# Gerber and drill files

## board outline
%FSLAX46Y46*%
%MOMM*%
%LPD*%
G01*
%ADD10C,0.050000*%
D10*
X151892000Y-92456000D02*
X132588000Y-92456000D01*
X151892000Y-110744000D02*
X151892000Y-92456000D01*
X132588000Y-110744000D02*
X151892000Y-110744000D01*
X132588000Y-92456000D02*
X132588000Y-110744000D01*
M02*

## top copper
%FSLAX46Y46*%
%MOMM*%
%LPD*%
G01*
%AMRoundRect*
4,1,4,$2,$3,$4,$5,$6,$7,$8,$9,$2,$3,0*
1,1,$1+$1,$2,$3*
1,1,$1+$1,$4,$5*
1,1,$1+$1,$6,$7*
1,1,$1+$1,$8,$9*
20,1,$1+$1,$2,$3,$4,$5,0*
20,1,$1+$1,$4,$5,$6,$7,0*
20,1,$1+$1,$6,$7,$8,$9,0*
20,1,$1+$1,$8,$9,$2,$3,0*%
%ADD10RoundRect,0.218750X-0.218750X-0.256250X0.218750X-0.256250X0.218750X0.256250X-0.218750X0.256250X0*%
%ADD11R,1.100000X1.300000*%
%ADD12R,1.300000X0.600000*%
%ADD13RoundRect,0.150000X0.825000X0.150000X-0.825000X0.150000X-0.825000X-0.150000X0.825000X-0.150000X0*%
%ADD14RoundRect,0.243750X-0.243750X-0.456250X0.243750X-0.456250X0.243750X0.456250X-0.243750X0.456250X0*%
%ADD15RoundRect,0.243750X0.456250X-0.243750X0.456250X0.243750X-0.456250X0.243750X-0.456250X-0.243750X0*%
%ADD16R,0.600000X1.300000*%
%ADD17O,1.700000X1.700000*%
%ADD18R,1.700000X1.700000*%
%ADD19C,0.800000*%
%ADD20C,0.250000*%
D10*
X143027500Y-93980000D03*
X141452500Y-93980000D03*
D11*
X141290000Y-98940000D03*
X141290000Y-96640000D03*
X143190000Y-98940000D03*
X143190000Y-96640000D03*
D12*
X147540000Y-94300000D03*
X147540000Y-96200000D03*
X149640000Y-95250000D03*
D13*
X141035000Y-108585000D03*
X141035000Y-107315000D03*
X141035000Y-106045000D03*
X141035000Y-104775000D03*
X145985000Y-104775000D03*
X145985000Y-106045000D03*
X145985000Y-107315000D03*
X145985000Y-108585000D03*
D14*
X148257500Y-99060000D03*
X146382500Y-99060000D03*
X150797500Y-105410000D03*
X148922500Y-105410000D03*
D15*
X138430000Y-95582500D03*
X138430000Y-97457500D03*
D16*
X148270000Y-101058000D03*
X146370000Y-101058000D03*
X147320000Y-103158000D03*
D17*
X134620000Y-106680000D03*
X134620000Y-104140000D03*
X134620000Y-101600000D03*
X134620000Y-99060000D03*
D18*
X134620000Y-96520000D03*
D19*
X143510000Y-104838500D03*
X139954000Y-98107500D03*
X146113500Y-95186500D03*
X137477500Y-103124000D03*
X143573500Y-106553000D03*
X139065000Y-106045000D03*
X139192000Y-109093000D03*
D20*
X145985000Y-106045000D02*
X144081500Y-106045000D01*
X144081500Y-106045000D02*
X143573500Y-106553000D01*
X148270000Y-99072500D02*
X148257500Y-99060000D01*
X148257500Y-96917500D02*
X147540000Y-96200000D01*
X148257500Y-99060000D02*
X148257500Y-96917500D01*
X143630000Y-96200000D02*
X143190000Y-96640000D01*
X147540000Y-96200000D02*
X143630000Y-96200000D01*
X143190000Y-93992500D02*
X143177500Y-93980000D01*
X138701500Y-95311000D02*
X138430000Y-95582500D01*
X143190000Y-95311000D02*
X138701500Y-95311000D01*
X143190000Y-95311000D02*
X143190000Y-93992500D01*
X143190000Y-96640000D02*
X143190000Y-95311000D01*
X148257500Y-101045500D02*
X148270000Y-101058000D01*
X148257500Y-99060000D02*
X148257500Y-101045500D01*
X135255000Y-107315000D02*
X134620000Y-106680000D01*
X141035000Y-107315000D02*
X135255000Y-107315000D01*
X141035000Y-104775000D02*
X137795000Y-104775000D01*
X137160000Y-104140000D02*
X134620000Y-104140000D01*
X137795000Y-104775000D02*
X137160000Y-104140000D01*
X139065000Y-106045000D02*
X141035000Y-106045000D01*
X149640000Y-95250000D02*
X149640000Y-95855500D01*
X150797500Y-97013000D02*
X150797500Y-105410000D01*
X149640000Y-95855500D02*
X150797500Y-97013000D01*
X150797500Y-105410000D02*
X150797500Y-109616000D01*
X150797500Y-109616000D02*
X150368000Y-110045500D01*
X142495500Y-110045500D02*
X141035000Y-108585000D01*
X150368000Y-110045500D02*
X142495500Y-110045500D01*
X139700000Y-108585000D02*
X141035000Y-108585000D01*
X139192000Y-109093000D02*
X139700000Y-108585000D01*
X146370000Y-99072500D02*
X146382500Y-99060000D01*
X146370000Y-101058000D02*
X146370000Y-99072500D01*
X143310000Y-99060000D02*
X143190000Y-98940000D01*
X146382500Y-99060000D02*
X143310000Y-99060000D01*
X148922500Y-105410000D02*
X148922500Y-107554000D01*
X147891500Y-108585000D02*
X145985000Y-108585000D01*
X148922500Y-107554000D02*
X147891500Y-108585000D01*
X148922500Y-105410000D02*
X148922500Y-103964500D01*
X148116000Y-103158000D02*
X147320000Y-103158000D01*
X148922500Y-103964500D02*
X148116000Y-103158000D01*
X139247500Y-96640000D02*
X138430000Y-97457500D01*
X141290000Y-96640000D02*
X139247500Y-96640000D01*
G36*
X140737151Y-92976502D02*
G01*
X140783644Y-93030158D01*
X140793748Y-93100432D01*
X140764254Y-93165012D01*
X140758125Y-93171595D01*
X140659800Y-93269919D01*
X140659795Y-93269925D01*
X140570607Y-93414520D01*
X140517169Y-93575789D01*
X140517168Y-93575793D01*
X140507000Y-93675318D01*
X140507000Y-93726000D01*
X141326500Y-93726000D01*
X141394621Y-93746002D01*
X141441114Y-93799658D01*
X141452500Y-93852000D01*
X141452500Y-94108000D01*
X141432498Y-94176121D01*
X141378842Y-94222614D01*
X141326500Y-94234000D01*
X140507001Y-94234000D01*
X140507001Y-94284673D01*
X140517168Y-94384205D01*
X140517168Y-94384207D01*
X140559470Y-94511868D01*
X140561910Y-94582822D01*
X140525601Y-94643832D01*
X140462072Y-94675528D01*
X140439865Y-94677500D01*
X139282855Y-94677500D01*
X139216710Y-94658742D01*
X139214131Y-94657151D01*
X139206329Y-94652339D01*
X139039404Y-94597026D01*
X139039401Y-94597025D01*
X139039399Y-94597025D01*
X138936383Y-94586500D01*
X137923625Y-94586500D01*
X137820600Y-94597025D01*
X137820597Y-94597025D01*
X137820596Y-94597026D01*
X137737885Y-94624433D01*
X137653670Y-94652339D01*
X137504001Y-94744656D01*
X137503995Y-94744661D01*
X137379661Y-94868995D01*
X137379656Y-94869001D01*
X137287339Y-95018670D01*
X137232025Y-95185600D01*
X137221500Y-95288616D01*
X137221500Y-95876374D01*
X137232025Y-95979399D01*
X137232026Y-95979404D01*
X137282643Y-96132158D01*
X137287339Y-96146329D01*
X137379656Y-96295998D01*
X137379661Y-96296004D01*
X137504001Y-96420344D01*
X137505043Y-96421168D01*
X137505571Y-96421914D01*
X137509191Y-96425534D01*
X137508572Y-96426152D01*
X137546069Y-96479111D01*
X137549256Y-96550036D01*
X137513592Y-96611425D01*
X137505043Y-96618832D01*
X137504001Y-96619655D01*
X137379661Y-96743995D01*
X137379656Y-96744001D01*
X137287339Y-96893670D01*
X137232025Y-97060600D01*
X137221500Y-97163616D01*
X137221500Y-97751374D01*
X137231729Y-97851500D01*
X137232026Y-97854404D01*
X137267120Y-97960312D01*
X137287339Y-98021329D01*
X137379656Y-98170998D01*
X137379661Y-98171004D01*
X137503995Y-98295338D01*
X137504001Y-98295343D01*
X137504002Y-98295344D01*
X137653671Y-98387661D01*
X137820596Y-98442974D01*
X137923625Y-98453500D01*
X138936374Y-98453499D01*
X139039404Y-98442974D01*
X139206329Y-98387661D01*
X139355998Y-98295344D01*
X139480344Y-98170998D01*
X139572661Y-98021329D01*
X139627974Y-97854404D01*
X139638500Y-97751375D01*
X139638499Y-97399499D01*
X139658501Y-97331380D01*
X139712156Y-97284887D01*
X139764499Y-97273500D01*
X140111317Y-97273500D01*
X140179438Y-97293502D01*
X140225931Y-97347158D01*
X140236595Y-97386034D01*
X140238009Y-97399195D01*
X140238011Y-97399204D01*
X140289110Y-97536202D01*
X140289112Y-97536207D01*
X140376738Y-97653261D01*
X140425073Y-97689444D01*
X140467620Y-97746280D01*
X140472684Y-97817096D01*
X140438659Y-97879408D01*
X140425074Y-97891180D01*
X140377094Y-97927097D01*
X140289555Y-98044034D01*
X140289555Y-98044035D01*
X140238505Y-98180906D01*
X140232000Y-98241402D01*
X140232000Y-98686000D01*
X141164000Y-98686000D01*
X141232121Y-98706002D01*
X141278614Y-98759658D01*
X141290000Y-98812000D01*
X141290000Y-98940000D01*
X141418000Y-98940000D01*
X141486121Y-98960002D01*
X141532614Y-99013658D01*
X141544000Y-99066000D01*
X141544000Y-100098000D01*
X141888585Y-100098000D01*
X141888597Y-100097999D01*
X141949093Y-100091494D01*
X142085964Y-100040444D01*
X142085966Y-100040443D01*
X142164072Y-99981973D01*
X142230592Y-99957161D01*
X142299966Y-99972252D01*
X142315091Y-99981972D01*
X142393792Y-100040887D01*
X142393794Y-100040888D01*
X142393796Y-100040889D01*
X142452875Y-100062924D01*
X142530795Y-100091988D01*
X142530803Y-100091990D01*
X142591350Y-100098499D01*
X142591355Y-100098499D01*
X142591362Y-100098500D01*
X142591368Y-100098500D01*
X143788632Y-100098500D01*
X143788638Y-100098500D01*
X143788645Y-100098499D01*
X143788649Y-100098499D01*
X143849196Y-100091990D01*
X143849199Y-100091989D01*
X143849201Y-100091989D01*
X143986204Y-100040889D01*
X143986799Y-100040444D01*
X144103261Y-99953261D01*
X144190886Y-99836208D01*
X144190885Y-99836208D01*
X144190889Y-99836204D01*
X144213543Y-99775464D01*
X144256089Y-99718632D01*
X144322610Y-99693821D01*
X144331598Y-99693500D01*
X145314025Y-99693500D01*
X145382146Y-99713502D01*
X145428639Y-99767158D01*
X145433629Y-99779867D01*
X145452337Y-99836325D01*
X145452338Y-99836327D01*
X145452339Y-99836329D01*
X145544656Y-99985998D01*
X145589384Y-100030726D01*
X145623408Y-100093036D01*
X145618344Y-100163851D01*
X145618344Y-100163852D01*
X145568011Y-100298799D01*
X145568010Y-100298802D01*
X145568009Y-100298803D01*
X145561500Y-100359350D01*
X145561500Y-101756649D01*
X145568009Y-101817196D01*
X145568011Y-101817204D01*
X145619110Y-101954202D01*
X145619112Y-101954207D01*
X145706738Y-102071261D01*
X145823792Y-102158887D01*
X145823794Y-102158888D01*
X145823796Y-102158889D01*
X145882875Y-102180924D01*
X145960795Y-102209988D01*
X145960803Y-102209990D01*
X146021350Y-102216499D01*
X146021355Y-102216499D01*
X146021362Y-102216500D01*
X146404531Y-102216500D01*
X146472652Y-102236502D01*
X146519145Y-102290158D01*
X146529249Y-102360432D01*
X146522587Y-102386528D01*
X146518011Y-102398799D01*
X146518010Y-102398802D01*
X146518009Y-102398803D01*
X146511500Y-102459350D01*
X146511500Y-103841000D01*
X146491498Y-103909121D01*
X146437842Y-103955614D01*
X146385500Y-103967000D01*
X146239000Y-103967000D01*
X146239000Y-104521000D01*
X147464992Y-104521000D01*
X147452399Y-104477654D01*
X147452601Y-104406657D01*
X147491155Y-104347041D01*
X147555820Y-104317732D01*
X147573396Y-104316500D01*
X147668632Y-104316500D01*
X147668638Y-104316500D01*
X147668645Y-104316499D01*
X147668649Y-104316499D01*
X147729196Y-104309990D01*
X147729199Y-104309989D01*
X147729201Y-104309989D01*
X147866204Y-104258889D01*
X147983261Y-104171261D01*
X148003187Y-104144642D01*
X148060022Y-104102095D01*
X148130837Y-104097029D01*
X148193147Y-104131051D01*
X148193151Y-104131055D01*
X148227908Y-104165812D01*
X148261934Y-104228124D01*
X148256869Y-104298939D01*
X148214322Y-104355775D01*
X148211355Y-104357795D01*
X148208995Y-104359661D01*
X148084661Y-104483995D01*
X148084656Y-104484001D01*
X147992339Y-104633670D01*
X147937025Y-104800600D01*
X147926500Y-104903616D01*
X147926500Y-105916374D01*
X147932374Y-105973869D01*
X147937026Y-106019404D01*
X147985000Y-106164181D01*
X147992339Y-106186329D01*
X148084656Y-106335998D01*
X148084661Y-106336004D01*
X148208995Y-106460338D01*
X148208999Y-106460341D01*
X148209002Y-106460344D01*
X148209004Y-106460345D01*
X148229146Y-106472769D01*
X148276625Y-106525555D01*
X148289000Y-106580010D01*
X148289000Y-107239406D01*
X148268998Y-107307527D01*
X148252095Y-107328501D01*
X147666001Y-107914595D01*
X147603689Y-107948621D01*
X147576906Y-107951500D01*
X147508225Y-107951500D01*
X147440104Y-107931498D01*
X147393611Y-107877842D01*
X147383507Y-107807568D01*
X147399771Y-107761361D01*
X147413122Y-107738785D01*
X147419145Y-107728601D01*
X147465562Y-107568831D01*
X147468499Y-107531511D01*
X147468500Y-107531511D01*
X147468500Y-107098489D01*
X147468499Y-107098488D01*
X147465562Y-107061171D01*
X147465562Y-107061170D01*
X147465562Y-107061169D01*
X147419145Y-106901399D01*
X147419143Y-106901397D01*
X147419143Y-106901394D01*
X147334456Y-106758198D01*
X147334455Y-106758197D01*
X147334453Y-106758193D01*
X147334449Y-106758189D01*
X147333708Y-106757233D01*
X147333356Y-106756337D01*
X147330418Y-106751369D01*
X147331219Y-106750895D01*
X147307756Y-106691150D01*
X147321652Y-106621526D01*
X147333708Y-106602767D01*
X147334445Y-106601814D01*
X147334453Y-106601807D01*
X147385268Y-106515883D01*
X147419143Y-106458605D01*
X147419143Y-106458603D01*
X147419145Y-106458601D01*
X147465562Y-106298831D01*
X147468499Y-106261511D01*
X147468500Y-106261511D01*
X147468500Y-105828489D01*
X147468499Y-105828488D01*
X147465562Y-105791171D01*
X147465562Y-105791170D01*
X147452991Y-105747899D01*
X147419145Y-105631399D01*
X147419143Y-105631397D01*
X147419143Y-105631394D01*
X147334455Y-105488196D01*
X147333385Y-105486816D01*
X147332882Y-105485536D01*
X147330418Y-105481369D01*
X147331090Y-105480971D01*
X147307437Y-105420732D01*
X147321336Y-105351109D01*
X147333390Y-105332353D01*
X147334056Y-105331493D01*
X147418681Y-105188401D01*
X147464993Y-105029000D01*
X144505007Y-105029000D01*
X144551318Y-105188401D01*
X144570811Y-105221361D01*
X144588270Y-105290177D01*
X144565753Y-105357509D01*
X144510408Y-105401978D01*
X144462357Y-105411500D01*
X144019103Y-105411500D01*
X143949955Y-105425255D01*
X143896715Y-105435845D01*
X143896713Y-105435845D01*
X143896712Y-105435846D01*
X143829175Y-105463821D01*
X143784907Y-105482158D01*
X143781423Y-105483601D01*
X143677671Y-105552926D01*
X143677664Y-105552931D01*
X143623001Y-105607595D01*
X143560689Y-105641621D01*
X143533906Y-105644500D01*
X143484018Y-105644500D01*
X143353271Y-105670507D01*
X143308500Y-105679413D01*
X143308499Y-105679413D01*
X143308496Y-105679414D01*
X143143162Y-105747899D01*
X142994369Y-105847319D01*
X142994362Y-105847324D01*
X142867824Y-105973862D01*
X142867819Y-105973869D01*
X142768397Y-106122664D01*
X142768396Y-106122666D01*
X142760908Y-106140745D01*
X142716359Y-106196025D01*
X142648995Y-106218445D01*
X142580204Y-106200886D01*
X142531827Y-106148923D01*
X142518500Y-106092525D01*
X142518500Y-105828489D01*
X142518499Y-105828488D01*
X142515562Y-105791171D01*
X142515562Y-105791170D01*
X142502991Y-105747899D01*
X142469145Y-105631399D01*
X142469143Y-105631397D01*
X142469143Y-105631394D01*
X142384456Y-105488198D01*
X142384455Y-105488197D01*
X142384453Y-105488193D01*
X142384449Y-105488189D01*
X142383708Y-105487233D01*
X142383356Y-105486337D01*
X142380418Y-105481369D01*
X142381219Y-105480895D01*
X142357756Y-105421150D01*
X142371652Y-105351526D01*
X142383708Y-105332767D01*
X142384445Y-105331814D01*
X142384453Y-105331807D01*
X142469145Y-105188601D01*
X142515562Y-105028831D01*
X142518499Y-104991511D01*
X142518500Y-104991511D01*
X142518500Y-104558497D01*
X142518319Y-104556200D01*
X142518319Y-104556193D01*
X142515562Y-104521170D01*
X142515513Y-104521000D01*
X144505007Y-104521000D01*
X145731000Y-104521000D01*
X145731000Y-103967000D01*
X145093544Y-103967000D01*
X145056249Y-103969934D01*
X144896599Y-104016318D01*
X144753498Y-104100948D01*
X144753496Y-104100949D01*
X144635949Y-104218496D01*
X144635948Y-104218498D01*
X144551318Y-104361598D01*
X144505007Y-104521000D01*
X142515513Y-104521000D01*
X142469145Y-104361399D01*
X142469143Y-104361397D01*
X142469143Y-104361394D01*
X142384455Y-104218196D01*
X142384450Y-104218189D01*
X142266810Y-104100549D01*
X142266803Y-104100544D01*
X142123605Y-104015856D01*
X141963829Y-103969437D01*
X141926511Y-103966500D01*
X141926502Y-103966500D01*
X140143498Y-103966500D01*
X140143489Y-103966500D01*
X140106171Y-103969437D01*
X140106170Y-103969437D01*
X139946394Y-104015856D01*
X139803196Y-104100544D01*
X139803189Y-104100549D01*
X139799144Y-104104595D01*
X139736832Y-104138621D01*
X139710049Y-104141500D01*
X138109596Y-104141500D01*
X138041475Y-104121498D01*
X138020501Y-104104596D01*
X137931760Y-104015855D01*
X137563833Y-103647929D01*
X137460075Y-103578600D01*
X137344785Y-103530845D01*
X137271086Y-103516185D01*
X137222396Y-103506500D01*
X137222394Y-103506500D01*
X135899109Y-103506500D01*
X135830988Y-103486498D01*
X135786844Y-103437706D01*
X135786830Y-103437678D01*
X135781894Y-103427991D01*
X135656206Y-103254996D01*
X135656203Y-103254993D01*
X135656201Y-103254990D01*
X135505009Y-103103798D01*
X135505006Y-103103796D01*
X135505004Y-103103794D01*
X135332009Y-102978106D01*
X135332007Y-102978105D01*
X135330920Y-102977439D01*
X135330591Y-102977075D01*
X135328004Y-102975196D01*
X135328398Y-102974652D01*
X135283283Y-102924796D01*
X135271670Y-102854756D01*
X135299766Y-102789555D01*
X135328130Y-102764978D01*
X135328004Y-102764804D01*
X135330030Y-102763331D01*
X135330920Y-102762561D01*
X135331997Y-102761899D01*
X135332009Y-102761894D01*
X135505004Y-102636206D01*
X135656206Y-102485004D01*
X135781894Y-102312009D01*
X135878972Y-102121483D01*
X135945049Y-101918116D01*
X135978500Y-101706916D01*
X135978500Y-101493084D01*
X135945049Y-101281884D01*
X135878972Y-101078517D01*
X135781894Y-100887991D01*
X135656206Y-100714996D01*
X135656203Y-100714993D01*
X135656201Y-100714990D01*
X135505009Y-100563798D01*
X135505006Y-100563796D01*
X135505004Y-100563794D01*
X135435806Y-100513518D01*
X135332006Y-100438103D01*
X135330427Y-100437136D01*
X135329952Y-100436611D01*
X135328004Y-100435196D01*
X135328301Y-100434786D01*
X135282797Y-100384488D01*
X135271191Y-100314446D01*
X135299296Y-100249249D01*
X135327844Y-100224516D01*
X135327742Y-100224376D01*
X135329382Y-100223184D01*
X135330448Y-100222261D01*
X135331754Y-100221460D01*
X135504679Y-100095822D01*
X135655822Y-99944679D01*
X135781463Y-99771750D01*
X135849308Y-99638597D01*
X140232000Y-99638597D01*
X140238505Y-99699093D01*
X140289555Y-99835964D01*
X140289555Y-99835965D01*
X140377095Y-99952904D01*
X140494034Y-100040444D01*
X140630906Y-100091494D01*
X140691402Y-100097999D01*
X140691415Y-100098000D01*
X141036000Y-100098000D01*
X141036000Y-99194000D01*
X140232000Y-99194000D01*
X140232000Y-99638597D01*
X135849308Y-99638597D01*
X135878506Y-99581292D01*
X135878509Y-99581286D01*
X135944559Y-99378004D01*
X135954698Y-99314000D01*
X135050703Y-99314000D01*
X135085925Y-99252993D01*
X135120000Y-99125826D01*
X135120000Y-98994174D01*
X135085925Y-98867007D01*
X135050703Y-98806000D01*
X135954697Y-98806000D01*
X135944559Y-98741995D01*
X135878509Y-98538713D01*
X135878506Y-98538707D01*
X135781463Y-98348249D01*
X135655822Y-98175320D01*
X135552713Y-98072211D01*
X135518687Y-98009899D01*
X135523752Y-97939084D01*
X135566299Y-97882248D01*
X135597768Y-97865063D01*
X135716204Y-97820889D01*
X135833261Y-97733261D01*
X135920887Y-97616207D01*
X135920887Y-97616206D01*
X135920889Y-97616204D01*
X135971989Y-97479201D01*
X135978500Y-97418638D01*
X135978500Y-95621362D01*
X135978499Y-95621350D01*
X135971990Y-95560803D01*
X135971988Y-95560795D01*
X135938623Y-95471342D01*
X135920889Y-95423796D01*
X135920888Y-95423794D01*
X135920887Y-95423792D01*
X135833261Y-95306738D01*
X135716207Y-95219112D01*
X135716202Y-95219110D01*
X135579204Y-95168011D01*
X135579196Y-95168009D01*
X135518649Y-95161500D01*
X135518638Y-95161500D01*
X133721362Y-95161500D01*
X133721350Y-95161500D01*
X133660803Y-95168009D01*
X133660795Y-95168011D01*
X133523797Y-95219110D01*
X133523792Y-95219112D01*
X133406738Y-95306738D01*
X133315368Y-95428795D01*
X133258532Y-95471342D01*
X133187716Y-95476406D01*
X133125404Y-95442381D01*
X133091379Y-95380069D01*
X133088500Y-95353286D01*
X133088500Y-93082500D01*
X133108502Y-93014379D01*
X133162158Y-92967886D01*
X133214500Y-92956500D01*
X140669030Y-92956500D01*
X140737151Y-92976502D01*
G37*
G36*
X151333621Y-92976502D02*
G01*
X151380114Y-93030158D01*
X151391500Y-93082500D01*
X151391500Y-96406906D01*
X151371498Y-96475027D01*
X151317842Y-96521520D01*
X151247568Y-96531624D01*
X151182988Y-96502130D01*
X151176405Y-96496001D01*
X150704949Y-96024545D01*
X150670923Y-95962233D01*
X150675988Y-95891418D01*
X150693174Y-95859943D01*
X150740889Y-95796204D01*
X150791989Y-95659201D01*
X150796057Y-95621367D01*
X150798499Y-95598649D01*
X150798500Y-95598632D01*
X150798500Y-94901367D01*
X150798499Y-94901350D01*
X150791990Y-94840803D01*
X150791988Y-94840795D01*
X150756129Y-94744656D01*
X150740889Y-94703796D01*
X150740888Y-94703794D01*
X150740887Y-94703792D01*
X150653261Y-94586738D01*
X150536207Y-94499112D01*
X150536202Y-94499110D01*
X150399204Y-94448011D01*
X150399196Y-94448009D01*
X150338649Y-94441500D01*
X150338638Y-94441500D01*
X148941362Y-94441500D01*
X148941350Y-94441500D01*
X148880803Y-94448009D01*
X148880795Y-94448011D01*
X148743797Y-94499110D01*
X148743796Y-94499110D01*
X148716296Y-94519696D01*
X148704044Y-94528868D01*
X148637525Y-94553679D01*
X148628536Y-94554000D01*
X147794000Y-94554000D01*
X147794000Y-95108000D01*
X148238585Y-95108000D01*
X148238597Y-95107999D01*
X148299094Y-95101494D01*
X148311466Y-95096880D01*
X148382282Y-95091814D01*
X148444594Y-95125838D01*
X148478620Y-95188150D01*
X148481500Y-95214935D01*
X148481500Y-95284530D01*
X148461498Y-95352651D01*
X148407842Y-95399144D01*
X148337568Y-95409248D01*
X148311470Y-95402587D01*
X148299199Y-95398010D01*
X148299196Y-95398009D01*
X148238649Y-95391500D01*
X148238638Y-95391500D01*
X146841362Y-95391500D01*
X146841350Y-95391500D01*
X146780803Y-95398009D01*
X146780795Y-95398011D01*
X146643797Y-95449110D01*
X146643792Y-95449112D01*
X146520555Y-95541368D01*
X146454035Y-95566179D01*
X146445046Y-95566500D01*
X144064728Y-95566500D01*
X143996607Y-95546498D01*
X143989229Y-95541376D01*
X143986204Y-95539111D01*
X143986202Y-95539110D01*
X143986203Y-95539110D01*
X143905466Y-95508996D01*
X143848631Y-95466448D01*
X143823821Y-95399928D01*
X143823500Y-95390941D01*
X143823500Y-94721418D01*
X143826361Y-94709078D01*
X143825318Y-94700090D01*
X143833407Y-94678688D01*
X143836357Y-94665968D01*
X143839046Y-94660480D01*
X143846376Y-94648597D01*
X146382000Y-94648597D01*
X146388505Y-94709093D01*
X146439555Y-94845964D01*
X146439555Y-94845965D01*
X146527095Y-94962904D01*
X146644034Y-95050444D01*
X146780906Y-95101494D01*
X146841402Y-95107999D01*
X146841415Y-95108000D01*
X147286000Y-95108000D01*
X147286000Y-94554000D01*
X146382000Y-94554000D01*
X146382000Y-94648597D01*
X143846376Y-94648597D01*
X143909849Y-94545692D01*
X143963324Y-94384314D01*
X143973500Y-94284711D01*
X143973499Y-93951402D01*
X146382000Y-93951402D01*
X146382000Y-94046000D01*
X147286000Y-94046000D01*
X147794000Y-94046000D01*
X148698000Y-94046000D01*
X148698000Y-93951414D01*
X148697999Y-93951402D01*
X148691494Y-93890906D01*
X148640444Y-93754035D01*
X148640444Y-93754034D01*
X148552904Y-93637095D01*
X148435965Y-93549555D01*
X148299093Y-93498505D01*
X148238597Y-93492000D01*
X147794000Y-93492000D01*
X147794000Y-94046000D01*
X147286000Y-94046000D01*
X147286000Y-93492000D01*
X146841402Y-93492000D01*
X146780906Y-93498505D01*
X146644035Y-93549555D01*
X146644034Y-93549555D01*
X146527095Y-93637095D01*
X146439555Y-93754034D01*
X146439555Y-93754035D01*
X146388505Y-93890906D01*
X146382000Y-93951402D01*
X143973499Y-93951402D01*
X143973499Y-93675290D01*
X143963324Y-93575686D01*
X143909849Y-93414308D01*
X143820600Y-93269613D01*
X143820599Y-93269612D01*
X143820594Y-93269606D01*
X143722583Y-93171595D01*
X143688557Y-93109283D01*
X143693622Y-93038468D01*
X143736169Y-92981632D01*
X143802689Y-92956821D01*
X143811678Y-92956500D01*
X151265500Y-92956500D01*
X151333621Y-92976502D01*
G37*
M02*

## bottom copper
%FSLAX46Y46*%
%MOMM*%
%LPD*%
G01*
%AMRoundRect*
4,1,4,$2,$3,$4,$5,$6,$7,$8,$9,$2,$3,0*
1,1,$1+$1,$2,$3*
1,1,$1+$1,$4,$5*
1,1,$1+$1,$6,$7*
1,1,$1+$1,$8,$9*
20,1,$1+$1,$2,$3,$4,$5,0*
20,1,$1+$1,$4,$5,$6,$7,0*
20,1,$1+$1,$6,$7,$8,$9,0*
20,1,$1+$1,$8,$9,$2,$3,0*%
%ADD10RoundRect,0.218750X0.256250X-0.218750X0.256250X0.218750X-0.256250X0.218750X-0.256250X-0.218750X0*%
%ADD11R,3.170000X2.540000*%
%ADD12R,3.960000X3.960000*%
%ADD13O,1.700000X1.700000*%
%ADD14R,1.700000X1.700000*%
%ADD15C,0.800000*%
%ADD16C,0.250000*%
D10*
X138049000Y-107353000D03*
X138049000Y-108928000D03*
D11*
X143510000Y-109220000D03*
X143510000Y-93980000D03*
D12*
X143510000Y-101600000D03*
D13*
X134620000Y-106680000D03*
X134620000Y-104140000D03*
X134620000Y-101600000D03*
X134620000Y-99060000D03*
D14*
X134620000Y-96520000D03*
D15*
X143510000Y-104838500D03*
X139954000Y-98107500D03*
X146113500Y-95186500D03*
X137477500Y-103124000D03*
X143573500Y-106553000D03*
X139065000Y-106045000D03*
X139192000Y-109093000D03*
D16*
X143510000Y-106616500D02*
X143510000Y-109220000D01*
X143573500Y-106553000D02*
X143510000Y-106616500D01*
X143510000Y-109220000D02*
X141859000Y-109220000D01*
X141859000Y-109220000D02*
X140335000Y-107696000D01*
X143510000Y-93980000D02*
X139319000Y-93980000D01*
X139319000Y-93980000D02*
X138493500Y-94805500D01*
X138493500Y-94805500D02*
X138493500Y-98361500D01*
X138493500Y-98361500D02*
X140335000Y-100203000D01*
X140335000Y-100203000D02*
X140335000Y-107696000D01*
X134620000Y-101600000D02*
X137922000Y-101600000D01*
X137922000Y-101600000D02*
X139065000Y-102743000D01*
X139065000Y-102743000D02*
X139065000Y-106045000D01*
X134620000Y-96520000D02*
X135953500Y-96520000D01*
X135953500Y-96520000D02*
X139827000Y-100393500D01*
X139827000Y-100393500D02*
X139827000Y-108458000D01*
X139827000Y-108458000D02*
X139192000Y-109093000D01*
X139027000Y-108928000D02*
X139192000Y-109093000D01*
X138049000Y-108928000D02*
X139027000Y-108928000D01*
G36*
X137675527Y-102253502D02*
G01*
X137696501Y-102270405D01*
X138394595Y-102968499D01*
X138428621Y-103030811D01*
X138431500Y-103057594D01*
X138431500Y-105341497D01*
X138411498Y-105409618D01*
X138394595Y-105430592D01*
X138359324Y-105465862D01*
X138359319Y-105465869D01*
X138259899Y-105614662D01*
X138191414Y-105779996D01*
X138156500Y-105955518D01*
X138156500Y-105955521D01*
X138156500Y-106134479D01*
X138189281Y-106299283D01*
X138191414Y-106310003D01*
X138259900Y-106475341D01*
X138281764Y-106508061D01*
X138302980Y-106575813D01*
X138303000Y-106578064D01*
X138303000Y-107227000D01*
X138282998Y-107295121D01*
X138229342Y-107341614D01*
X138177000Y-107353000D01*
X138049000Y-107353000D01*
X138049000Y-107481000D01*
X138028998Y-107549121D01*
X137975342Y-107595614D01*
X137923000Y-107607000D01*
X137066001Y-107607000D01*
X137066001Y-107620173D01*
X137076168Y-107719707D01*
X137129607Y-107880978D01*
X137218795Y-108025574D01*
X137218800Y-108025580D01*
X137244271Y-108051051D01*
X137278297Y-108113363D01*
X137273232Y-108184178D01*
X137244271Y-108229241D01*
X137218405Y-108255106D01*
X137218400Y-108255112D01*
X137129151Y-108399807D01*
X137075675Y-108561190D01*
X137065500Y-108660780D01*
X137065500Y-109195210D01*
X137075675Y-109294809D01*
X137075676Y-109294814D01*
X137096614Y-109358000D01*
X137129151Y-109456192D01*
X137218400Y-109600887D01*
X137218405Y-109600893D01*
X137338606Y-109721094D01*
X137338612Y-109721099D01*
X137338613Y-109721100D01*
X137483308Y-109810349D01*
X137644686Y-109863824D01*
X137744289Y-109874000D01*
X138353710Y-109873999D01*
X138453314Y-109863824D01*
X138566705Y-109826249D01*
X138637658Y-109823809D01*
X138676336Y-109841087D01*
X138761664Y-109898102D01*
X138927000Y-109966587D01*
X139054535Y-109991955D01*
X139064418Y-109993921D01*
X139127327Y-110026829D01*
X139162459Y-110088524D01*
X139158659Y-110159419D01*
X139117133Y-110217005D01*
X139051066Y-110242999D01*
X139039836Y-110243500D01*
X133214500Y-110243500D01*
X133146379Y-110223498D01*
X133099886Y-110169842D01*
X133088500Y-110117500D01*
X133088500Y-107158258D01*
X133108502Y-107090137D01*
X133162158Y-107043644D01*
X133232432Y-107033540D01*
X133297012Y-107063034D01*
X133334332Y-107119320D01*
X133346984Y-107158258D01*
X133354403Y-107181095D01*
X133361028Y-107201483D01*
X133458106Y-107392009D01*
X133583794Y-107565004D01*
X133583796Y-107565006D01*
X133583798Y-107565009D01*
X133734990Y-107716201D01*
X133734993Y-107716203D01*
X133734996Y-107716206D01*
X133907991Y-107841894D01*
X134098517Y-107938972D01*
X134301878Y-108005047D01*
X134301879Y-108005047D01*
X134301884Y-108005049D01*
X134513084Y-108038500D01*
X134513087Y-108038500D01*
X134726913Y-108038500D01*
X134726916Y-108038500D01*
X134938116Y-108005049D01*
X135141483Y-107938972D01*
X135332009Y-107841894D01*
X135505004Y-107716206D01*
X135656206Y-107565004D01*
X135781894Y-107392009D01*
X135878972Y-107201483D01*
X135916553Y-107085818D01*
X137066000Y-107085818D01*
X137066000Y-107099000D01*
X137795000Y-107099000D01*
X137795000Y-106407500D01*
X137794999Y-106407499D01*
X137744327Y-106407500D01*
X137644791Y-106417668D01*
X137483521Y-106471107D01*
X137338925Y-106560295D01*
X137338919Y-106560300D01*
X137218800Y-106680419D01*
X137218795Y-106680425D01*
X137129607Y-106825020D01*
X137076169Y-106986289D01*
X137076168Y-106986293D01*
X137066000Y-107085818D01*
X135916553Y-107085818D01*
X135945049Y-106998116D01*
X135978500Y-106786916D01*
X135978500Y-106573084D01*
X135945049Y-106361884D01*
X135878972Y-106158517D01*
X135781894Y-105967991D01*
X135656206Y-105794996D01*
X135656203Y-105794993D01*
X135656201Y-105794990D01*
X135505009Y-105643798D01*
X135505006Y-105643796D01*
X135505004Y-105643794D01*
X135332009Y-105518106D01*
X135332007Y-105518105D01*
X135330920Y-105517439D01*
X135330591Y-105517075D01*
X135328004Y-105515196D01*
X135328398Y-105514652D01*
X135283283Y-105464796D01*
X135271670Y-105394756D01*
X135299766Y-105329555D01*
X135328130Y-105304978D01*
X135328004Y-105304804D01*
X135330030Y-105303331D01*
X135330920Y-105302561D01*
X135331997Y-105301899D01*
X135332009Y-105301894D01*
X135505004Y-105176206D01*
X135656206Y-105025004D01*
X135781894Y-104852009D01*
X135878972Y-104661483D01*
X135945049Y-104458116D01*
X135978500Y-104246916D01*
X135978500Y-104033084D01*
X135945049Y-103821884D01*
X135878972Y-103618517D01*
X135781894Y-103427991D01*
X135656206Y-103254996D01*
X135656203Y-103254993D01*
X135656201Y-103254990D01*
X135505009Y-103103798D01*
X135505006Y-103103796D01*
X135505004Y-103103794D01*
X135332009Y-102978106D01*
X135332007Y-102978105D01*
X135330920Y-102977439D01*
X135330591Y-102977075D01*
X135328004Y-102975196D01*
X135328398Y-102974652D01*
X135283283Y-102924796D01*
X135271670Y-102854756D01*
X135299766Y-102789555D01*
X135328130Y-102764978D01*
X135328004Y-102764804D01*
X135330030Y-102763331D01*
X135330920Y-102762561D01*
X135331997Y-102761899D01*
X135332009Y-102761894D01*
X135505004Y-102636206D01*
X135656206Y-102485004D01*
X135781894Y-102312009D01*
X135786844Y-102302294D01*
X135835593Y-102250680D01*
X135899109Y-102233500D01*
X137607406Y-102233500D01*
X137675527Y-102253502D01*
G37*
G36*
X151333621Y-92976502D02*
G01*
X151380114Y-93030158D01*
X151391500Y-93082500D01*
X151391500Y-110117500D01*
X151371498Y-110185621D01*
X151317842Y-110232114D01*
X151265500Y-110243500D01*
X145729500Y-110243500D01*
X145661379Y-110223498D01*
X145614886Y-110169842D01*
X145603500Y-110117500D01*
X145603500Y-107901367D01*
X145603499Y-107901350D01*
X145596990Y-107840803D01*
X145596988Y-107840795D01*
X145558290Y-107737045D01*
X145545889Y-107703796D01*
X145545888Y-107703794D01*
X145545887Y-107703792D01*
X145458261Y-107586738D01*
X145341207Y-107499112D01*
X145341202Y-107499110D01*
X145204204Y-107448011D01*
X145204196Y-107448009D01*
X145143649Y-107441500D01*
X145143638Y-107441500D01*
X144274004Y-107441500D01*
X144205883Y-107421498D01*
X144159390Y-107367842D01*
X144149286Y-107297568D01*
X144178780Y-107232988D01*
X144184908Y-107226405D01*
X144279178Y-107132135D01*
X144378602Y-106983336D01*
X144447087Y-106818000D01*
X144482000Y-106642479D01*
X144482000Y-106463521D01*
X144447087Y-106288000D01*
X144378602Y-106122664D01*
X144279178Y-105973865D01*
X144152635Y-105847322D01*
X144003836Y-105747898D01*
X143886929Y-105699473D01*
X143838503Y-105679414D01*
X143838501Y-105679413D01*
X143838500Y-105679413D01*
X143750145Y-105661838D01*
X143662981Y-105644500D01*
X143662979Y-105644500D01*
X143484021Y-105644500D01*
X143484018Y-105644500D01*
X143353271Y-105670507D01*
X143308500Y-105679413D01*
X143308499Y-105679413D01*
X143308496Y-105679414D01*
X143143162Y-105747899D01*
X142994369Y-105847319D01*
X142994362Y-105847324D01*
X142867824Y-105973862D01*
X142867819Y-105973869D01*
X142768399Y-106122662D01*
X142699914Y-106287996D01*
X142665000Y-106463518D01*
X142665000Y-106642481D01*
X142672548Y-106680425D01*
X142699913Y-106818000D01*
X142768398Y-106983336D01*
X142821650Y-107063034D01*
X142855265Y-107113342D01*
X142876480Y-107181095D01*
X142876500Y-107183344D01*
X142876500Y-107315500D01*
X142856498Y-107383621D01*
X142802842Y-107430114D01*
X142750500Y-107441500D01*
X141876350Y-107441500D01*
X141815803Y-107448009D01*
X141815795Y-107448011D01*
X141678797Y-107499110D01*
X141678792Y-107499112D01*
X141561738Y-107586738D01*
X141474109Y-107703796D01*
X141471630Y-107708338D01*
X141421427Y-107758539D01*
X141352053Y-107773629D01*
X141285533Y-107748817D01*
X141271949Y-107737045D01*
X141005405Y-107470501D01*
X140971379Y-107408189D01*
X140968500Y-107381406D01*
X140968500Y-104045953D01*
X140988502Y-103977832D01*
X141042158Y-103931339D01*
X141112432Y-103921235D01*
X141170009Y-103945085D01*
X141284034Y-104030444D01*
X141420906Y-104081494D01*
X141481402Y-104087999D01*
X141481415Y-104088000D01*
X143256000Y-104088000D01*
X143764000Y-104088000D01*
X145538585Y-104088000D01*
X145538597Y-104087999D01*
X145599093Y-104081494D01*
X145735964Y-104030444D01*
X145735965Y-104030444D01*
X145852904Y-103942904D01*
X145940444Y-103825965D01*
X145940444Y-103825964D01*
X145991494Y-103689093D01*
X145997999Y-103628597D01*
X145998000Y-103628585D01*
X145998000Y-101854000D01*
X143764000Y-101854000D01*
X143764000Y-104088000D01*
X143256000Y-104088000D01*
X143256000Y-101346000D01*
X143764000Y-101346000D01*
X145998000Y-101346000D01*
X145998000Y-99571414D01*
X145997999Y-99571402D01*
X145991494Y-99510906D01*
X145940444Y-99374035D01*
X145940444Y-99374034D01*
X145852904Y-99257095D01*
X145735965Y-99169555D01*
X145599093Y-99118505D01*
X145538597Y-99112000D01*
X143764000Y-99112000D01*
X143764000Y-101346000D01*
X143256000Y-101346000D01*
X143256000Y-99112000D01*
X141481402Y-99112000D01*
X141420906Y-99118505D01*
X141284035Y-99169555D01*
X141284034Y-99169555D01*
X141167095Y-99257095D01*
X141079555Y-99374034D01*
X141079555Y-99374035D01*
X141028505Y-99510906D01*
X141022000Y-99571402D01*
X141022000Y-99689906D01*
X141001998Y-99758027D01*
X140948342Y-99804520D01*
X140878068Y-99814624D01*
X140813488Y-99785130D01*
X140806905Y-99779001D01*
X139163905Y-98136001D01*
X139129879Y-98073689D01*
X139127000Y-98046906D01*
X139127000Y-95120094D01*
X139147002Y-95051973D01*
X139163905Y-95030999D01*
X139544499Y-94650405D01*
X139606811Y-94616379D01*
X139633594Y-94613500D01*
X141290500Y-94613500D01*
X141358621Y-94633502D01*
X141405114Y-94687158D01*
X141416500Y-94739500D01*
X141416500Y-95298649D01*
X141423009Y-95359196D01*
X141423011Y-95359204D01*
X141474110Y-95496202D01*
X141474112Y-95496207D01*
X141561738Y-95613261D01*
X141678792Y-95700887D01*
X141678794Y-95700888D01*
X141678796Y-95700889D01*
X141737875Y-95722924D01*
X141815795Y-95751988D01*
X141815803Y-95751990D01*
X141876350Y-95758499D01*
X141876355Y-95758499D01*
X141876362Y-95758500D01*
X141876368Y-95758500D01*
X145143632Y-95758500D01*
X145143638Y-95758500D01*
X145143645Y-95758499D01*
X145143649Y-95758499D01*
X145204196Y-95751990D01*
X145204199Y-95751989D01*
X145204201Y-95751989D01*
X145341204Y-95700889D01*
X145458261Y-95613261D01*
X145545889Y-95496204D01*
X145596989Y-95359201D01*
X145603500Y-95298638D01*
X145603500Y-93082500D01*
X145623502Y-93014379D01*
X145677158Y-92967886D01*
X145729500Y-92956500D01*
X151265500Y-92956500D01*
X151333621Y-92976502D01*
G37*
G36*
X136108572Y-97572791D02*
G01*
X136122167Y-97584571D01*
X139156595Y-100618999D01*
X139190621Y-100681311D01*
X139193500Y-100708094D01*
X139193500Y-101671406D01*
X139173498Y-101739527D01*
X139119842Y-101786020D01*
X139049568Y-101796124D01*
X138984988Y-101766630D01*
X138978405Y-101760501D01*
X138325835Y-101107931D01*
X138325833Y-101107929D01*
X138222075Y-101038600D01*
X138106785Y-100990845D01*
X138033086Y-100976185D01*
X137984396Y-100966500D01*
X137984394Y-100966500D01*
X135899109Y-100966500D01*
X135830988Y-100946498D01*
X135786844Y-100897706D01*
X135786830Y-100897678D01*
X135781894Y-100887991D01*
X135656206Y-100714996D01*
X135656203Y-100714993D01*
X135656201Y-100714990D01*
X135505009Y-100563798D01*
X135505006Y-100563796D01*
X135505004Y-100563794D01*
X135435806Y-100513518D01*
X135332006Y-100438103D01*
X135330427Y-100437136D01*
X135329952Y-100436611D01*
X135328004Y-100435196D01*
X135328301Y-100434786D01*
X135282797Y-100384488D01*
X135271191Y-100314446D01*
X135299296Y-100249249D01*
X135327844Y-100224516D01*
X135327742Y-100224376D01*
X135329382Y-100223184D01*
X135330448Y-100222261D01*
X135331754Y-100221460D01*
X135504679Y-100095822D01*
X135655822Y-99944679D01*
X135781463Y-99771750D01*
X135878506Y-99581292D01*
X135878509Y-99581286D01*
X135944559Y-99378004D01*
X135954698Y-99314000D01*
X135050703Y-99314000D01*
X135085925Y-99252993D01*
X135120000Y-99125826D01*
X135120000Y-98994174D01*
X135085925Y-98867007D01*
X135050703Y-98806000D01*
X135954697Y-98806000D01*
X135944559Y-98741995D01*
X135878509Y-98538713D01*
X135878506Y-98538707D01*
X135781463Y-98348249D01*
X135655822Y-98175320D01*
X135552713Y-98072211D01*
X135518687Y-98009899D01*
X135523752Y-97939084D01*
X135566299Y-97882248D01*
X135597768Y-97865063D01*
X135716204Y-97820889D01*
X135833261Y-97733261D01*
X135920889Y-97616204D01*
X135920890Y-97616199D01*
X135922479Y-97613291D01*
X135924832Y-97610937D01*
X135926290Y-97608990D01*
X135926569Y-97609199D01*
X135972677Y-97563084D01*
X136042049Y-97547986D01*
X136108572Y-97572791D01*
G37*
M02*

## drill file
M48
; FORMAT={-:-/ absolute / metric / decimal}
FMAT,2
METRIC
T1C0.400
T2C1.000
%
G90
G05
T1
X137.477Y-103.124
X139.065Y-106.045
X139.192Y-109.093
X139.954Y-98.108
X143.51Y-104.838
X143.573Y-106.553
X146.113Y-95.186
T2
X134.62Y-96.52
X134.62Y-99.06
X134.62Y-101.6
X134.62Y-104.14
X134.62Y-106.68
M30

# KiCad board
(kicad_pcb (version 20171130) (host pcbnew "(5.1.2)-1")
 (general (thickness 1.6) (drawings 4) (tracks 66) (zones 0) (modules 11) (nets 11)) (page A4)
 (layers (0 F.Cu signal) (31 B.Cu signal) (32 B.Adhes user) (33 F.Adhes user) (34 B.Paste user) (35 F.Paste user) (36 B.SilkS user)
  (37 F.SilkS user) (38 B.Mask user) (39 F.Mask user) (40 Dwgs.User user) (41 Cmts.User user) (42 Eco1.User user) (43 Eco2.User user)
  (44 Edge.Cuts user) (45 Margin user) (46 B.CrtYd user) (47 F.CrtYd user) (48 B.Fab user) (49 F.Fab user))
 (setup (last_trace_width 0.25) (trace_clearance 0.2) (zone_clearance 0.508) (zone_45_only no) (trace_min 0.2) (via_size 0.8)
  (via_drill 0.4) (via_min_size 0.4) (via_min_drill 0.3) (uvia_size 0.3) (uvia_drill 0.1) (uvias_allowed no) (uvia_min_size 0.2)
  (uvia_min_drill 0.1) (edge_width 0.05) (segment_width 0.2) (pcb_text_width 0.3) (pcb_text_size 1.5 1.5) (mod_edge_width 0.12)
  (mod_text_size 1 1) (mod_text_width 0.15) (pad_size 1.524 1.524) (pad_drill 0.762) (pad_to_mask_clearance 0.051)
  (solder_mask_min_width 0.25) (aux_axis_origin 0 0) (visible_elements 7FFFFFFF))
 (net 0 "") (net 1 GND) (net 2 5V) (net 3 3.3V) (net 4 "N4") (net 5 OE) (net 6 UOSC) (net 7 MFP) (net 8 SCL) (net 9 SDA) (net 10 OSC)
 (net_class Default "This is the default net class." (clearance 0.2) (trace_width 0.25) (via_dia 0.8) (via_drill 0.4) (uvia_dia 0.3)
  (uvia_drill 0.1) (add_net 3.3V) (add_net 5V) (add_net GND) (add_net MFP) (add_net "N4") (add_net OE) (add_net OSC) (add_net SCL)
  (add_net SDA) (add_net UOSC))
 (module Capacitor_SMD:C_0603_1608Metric (layer B.Cu) (at 138.049 108.1405 90)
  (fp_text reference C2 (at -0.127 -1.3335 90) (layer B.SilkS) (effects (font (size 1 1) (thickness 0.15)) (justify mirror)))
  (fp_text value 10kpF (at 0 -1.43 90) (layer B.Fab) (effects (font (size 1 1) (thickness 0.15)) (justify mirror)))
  (pad 2 smd roundrect (at 0.7875 0 90) (size 0.875 0.95) (layers B.Cu B.Paste B.Mask) (roundrect_rratio 0.25) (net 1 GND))
  (pad 1 smd roundrect (at -0.7875 0 90) (size 0.875 0.95) (layers B.Cu B.Paste B.Mask) (roundrect_rratio 0.25) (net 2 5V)))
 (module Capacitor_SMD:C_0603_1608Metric (layer F.Cu) (at 142.24 93.98)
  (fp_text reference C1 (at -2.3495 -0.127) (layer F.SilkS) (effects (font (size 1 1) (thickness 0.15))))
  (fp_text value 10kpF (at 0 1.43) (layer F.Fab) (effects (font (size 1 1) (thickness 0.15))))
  (pad 2 smd roundrect (at 0.7875 0) (size 0.875 0.95) (layers F.Cu F.Paste F.Mask) (roundrect_rratio 0.25) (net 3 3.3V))
  (pad 1 smd roundrect (at -0.7875 0) (size 0.875 0.95) (layers F.Cu F.Paste F.Mask) (roundrect_rratio 0.25) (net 1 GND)))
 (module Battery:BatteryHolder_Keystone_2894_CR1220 (layer B.Cu) (at 143.51 101.6 270)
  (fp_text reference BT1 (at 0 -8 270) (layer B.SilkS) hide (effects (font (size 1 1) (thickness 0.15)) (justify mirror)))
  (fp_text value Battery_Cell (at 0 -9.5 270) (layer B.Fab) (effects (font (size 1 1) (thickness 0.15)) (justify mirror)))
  (pad 1 smd rect (at 7.62 0 270) (size 2.54 3.17) (layers B.Cu B.Paste B.Mask) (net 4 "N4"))
  (pad 1 smd rect (at -7.62 0 270) (size 2.54 3.17) (layers B.Cu B.Paste B.Mask) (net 4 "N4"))
  (pad 2 smd rect (at 0 0 270) (size 3.96 3.96) (layers B.Cu B.Paste B.Mask) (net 1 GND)))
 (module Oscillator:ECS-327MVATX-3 (layer F.Cu) (at 142.24 97.79 270)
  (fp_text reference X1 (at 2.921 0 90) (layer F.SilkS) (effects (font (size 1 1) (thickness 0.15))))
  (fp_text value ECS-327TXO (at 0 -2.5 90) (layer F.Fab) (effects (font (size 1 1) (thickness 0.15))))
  (pad 2 smd rect (at 1.15 0.95 270) (size 1.3 1.1) (layers F.Cu F.Paste F.Mask) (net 1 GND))
  (pad 1 smd rect (at -1.15 0.95 270) (size 1.3 1.1) (layers F.Cu F.Paste F.Mask) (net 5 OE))
  (pad 3 smd rect (at 1.15 -0.95 270) (size 1.3 1.1) (layers F.Cu F.Paste F.Mask) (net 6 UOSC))
  (pad 4 smd rect (at -1.15 -0.95 270) (size 1.3 1.1) (layers F.Cu F.Paste F.Mask) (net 3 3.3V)))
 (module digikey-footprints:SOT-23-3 (layer F.Cu) (at 148.59 95.25)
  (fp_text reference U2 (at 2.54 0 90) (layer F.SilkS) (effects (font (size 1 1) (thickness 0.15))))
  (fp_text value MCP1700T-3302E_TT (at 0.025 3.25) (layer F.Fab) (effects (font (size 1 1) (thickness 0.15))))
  (pad 1 smd rect (at -1.05 -0.95) (size 1.3 0.6) (layers F.Cu F.Paste F.Mask) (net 1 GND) (solder_mask_margin 0.07))
  (pad 2 smd rect (at -1.05 0.95) (size 1.3 0.6) (layers F.Cu F.Paste F.Mask) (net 3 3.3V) (solder_mask_margin 0.07))
  (pad 3 smd rect (at 1.05 0) (size 1.3 0.6) (layers F.Cu F.Paste F.Mask) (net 2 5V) (solder_mask_margin 0.07)))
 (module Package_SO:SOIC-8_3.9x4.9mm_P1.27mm (layer F.Cu) (at 143.51 106.68 180)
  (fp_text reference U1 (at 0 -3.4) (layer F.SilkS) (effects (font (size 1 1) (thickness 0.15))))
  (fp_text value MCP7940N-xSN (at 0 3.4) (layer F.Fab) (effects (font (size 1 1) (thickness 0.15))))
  (pad 8 smd roundrect (at 2.475 -1.905 180) (size 1.95 0.6) (layers F.Cu F.Paste F.Mask) (roundrect_rratio 0.25) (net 2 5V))
  (pad 7 smd roundrect (at 2.475 -0.635 180) (size 1.95 0.6) (layers F.Cu F.Paste F.Mask) (roundrect_rratio 0.25) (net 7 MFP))
  (pad 6 smd roundrect (at 2.475 0.635 180) (size 1.95 0.6) (layers F.Cu F.Paste F.Mask) (roundrect_rratio 0.25) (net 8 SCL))
  (pad 5 smd roundrect (at 2.475 1.905 180) (size 1.95 0.6) (layers F.Cu F.Paste F.Mask) (roundrect_rratio 0.25) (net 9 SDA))
  (pad 4 smd roundrect (at -2.475 1.905 180) (size 1.95 0.6) (layers F.Cu F.Paste F.Mask) (roundrect_rratio 0.25) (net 1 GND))
  (pad 3 smd roundrect (at -2.475 0.635 180) (size 1.95 0.6) (layers F.Cu F.Paste F.Mask) (roundrect_rratio 0.25) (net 4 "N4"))
  (pad 2 smd roundrect (at -2.475 -0.635 180) (size 1.95 0.6) (layers F.Cu F.Paste F.Mask) (roundrect_rratio 0.25))
  (pad 1 smd roundrect (at -2.475 -1.905 180) (size 1.95 0.6) (layers F.Cu F.Paste F.Mask) (roundrect_rratio 0.25) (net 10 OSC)))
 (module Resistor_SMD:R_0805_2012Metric (layer F.Cu) (at 147.32 99.06)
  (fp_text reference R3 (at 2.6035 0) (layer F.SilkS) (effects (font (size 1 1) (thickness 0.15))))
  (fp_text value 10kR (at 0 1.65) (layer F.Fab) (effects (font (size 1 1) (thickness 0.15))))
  (pad 2 smd roundrect (at 0.9375 0) (size 0.975 1.4) (layers F.Cu F.Paste F.Mask) (roundrect_rratio 0.25) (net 3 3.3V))
  (pad 1 smd roundrect (at -0.9375 0) (size 0.975 1.4) (layers F.Cu F.Paste F.Mask) (roundrect_rratio 0.25) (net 6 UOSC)))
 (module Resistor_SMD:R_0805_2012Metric (layer F.Cu) (at 149.86 105.41)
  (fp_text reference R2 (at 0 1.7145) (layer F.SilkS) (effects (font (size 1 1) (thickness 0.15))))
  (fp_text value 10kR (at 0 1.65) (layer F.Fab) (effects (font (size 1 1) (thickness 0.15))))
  (pad 2 smd roundrect (at 0.9375 0) (size 0.975 1.4) (layers F.Cu F.Paste F.Mask) (roundrect_rratio 0.25) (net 2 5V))
  (pad 1 smd roundrect (at -0.9375 0) (size 0.975 1.4) (layers F.Cu F.Paste F.Mask) (roundrect_rratio 0.25) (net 10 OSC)))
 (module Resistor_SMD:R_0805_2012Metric (layer F.Cu) (at 138.43 96.52 90)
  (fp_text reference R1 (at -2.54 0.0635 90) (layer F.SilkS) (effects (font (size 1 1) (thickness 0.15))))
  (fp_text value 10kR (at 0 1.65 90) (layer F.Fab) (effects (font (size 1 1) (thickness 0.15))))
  (pad 2 smd roundrect (at 0.9375 0 90) (size 0.975 1.4) (layers F.Cu F.Paste F.Mask) (roundrect_rratio 0.25) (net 3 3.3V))
  (pad 1 smd roundrect (at -0.9375 0 90) (size 0.975 1.4) (layers F.Cu F.Paste F.Mask) (roundrect_rratio 0.25) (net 5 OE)))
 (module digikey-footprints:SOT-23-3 (layer F.Cu) (at 147.32 102.108 270)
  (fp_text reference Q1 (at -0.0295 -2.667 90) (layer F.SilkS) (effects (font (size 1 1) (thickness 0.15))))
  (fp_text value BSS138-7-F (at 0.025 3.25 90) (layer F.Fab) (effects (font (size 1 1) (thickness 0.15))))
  (pad 1 smd rect (at -1.05 -0.95 270) (size 1.3 0.6) (layers F.Cu F.Paste F.Mask) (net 3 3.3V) (solder_mask_margin 0.07))
  (pad 2 smd rect (at -1.05 0.95 270) (size 1.3 0.6) (layers F.Cu F.Paste F.Mask) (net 6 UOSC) (solder_mask_margin 0.07))
  (pad 3 smd rect (at 1.05 0 270) (size 1.3 0.6) (layers F.Cu F.Paste F.Mask) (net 10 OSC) (solder_mask_margin 0.07)))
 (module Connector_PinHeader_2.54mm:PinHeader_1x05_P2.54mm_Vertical (layer B.Cu) (at 134.62 96.52 180)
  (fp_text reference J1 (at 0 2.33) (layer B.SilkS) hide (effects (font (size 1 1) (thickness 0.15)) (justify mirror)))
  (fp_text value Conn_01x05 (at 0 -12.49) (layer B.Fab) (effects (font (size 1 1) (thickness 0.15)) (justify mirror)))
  (pad 5 thru_hole oval (at 0 -10.16 180) (size 1.7 1.7) (drill 1) (layers *.Cu *.Mask) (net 7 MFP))
  (pad 4 thru_hole oval (at 0 -7.62 180) (size 1.7 1.7) (drill 1) (layers *.Cu *.Mask) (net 9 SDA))
  (pad 3 thru_hole oval (at 0 -5.08 180) (size 1.7 1.7) (drill 1) (layers *.Cu *.Mask) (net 8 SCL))
  (pad 2 thru_hole oval (at 0 -2.54 180) (size 1.7 1.7) (drill 1) (layers *.Cu *.Mask) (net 1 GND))
  (pad 1 thru_hole rect (at 0 0 180) (size 1.7 1.7) (drill 1) (layers *.Cu *.Mask) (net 2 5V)))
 (gr_line (start 151.892 92.456) (end 132.588 92.456) (layer Edge.Cuts) (width 0.05))
 (gr_line (start 151.892 110.744) (end 151.892 92.456) (layer Edge.Cuts) (width 0.05))
 (gr_line (start 132.588 110.744) (end 151.892 110.744) (layer Edge.Cuts) (width 0.05))
 (gr_line (start 132.588 92.456) (end 132.588 110.744) (layer Edge.Cuts) (width 0.05))
 (via (at 143.51 104.8385) (size 0.8) (drill 0.4) (layers F.Cu B.Cu) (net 1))
 (via (at 139.954 98.1075) (size 0.8) (drill 0.4) (layers F.Cu B.Cu) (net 1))
 (via (at 146.1135 95.1865) (size 0.8) (drill 0.4) (layers F.Cu B.Cu) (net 1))
 (via (at 137.4775 103.124) (size 0.8) (drill 0.4) (layers F.Cu B.Cu) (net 1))
 (via (at 143.5735 106.553) (size 0.8) (drill 0.4) (layers F.Cu B.Cu) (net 4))
 (segment (start 145.985 106.045) (end 144.0815 106.045) (width 0.25) (layer F.Cu) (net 4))
 (segment (start 144.0815 106.045) (end 143.5735 106.553) (width 0.25) (layer F.Cu) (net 4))
 (segment (start 143.51 106.6165) (end 143.51 109.22) (width 0.25) (layer B.Cu) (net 4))
 (segment (start 143.5735 106.553) (end 143.51 106.6165) (width 0.25) (layer B.Cu) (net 4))
 (segment (start 143.51 109.22) (end 141.859 109.22) (width 0.25) (layer B.Cu) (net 4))
 (segment (start 141.859 109.22) (end 140.335 107.696) (width 0.25) (layer B.Cu) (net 4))
 (segment (start 143.51 93.98) (end 139.319 93.98) (width 0.25) (layer B.Cu) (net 4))
 (segment (start 139.319 93.98) (end 138.4935 94.8055) (width 0.25) (layer B.Cu) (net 4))
 (segment (start 138.4935 94.8055) (end 138.4935 98.3615) (width 0.25) (layer B.Cu) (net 4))
 (segment (start 138.4935 98.3615) (end 140.335 100.203) (width 0.25) (layer B.Cu) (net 4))
 (segment (start 140.335 100.203) (end 140.335 107.696) (width 0.25) (layer B.Cu) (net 4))
 (segment (start 148.27 99.0725) (end 148.2575 99.06) (width 0.25) (layer F.Cu) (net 3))
 (segment (start 148.2575 96.9175) (end 147.54 96.2) (width 0.25) (layer F.Cu) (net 3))
 (segment (start 148.2575 99.06) (end 148.2575 96.9175) (width 0.25) (layer F.Cu) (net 3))
 (segment (start 143.63 96.2) (end 143.19 96.64) (width 0.25) (layer F.Cu) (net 3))
 (segment (start 147.54 96.2) (end 143.63 96.2) (width 0.25) (layer F.Cu) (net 3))
 (segment (start 143.19 93.9925) (end 143.1775 93.98) (width 0.25) (layer F.Cu) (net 3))
 (segment (start 138.7015 95.311) (end 138.43 95.5825) (width 0.25) (layer F.Cu) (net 3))
 (segment (start 143.19 95.311) (end 138.7015 95.311) (width 0.25) (layer F.Cu) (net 3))
 (segment (start 143.19 95.311) (end 143.19 93.9925) (width 0.25) (layer F.Cu) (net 3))
 (segment (start 143.19 96.64) (end 143.19 95.311) (width 0.25) (layer F.Cu) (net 3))
 (segment (start 148.2575 101.0455) (end 148.27 101.058) (width 0.25) (layer F.Cu) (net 3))
 (segment (start 148.2575 99.06) (end 148.2575 101.0455) (width 0.25) (layer F.Cu) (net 3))
 (segment (start 135.255 107.315) (end 134.62 106.68) (width 0.25) (layer F.Cu) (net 7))
 (segment (start 141.035 107.315) (end 135.255 107.315) (width 0.25) (layer F.Cu) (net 7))
 (segment (start 141.035 104.775) (end 137.795 104.775) (width 0.25) (layer F.Cu) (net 9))
 (segment (start 137.16 104.14) (end 134.62 104.14) (width 0.25) (layer F.Cu) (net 9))
 (segment (start 137.795 104.775) (end 137.16 104.14) (width 0.25) (layer F.Cu) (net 9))
 (segment (start 134.62 101.6) (end 137.922 101.6) (width 0.25) (layer B.Cu) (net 8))
 (via (at 139.065 106.045) (size 0.8) (drill 0.4) (layers F.Cu B.Cu) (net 8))
 (segment (start 137.922 101.6) (end 139.065 102.743) (width 0.25) (layer B.Cu) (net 8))
 (segment (start 139.065 102.743) (end 139.065 106.045) (width 0.25) (layer B.Cu) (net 8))
 (segment (start 139.065 106.045) (end 141.035 106.045) (width 0.25) (layer F.Cu) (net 8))
 (segment (start 149.64 95.25) (end 149.64 95.8555) (width 0.25) (layer F.Cu) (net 2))
 (segment (start 150.7975 97.013) (end 150.7975 105.41) (width 0.25) (layer F.Cu) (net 2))
 (segment (start 149.64 95.8555) (end 150.7975 97.013) (width 0.25) (layer F.Cu) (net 2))
 (segment (start 150.7975 105.41) (end 150.7975 109.616) (width 0.25) (layer F.Cu) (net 2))
 (segment (start 150.7975 109.616) (end 150.368 110.0455) (width 0.25) (layer F.Cu) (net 2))
 (segment (start 142.4955 110.0455) (end 141.035 108.585) (width 0.25) (layer F.Cu) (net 2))
 (segment (start 150.368 110.0455) (end 142.4955 110.0455) (width 0.25) (layer F.Cu) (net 2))
 (segment (start 134.62 96.52) (end 135.9535 96.52) (width 0.25) (layer B.Cu) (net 2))
 (segment (start 135.9535 96.52) (end 139.827 100.3935) (width 0.25) (layer B.Cu) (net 2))
 (via (at 139.192 109.093) (size 0.8) (drill 0.4) (layers F.Cu B.Cu) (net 2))
 (segment (start 139.827 100.3935) (end 139.827 108.458) (width 0.25) (layer B.Cu) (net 2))
 (segment (start 139.827 108.458) (end 139.192 109.093) (width 0.25) (layer B.Cu) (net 2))
 (segment (start 139.7 108.585) (end 141.035 108.585) (width 0.25) (layer F.Cu) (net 2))
 (segment (start 139.192 109.093) (end 139.7 108.585) (width 0.25) (layer F.Cu) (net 2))
 (segment (start 139.027 108.928) (end 139.192 109.093) (width 0.25) (layer B.Cu) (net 2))
 (segment (start 138.049 108.928) (end 139.027 108.928) (width 0.25) (layer B.Cu) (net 2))
 (segment (start 146.37 99.0725) (end 146.3825 99.06) (width 0.25) (layer F.Cu) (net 6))
 (segment (start 146.37 101.058) (end 146.37 99.0725) (width 0.25) (layer F.Cu) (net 6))
 (segment (start 143.31 99.06) (end 143.19 98.94) (width 0.25) (layer F.Cu) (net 6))
 (segment (start 146.3825 99.06) (end 143.31 99.06) (width 0.25) (layer F.Cu) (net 6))
 (segment (start 148.9225 105.41) (end 148.9225 107.554) (width 0.25) (layer F.Cu) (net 10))
 (segment (start 147.8915 108.585) (end 145.985 108.585) (width 0.25) (layer F.Cu) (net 10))
 (segment (start 148.9225 107.554) (end 147.8915 108.585) (width 0.25) (layer F.Cu) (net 10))
 (segment (start 148.9225 105.41) (end 148.9225 103.9645) (width 0.25) (layer F.Cu) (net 10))
 (segment (start 148.116 103.158) (end 147.32 103.158) (width 0.25) (layer F.Cu) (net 10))
 (segment (start 148.9225 103.9645) (end 148.116 103.158) (width 0.25) (layer F.Cu) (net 10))
 (segment (start 139.2475 96.64) (end 138.43 97.4575) (width 0.25) (layer F.Cu) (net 5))
 (segment (start 141.29 96.64) (end 139.2475 96.64) (width 0.25) (layer F.Cu) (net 5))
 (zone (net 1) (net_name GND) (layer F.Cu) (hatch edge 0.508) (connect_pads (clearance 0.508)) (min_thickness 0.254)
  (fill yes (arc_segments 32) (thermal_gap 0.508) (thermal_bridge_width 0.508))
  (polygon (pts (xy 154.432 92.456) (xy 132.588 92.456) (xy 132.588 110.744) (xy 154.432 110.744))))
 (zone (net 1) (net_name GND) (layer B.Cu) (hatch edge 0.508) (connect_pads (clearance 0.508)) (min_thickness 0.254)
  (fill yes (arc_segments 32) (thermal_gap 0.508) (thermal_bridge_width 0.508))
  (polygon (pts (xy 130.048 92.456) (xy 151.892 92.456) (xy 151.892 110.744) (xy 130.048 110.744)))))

